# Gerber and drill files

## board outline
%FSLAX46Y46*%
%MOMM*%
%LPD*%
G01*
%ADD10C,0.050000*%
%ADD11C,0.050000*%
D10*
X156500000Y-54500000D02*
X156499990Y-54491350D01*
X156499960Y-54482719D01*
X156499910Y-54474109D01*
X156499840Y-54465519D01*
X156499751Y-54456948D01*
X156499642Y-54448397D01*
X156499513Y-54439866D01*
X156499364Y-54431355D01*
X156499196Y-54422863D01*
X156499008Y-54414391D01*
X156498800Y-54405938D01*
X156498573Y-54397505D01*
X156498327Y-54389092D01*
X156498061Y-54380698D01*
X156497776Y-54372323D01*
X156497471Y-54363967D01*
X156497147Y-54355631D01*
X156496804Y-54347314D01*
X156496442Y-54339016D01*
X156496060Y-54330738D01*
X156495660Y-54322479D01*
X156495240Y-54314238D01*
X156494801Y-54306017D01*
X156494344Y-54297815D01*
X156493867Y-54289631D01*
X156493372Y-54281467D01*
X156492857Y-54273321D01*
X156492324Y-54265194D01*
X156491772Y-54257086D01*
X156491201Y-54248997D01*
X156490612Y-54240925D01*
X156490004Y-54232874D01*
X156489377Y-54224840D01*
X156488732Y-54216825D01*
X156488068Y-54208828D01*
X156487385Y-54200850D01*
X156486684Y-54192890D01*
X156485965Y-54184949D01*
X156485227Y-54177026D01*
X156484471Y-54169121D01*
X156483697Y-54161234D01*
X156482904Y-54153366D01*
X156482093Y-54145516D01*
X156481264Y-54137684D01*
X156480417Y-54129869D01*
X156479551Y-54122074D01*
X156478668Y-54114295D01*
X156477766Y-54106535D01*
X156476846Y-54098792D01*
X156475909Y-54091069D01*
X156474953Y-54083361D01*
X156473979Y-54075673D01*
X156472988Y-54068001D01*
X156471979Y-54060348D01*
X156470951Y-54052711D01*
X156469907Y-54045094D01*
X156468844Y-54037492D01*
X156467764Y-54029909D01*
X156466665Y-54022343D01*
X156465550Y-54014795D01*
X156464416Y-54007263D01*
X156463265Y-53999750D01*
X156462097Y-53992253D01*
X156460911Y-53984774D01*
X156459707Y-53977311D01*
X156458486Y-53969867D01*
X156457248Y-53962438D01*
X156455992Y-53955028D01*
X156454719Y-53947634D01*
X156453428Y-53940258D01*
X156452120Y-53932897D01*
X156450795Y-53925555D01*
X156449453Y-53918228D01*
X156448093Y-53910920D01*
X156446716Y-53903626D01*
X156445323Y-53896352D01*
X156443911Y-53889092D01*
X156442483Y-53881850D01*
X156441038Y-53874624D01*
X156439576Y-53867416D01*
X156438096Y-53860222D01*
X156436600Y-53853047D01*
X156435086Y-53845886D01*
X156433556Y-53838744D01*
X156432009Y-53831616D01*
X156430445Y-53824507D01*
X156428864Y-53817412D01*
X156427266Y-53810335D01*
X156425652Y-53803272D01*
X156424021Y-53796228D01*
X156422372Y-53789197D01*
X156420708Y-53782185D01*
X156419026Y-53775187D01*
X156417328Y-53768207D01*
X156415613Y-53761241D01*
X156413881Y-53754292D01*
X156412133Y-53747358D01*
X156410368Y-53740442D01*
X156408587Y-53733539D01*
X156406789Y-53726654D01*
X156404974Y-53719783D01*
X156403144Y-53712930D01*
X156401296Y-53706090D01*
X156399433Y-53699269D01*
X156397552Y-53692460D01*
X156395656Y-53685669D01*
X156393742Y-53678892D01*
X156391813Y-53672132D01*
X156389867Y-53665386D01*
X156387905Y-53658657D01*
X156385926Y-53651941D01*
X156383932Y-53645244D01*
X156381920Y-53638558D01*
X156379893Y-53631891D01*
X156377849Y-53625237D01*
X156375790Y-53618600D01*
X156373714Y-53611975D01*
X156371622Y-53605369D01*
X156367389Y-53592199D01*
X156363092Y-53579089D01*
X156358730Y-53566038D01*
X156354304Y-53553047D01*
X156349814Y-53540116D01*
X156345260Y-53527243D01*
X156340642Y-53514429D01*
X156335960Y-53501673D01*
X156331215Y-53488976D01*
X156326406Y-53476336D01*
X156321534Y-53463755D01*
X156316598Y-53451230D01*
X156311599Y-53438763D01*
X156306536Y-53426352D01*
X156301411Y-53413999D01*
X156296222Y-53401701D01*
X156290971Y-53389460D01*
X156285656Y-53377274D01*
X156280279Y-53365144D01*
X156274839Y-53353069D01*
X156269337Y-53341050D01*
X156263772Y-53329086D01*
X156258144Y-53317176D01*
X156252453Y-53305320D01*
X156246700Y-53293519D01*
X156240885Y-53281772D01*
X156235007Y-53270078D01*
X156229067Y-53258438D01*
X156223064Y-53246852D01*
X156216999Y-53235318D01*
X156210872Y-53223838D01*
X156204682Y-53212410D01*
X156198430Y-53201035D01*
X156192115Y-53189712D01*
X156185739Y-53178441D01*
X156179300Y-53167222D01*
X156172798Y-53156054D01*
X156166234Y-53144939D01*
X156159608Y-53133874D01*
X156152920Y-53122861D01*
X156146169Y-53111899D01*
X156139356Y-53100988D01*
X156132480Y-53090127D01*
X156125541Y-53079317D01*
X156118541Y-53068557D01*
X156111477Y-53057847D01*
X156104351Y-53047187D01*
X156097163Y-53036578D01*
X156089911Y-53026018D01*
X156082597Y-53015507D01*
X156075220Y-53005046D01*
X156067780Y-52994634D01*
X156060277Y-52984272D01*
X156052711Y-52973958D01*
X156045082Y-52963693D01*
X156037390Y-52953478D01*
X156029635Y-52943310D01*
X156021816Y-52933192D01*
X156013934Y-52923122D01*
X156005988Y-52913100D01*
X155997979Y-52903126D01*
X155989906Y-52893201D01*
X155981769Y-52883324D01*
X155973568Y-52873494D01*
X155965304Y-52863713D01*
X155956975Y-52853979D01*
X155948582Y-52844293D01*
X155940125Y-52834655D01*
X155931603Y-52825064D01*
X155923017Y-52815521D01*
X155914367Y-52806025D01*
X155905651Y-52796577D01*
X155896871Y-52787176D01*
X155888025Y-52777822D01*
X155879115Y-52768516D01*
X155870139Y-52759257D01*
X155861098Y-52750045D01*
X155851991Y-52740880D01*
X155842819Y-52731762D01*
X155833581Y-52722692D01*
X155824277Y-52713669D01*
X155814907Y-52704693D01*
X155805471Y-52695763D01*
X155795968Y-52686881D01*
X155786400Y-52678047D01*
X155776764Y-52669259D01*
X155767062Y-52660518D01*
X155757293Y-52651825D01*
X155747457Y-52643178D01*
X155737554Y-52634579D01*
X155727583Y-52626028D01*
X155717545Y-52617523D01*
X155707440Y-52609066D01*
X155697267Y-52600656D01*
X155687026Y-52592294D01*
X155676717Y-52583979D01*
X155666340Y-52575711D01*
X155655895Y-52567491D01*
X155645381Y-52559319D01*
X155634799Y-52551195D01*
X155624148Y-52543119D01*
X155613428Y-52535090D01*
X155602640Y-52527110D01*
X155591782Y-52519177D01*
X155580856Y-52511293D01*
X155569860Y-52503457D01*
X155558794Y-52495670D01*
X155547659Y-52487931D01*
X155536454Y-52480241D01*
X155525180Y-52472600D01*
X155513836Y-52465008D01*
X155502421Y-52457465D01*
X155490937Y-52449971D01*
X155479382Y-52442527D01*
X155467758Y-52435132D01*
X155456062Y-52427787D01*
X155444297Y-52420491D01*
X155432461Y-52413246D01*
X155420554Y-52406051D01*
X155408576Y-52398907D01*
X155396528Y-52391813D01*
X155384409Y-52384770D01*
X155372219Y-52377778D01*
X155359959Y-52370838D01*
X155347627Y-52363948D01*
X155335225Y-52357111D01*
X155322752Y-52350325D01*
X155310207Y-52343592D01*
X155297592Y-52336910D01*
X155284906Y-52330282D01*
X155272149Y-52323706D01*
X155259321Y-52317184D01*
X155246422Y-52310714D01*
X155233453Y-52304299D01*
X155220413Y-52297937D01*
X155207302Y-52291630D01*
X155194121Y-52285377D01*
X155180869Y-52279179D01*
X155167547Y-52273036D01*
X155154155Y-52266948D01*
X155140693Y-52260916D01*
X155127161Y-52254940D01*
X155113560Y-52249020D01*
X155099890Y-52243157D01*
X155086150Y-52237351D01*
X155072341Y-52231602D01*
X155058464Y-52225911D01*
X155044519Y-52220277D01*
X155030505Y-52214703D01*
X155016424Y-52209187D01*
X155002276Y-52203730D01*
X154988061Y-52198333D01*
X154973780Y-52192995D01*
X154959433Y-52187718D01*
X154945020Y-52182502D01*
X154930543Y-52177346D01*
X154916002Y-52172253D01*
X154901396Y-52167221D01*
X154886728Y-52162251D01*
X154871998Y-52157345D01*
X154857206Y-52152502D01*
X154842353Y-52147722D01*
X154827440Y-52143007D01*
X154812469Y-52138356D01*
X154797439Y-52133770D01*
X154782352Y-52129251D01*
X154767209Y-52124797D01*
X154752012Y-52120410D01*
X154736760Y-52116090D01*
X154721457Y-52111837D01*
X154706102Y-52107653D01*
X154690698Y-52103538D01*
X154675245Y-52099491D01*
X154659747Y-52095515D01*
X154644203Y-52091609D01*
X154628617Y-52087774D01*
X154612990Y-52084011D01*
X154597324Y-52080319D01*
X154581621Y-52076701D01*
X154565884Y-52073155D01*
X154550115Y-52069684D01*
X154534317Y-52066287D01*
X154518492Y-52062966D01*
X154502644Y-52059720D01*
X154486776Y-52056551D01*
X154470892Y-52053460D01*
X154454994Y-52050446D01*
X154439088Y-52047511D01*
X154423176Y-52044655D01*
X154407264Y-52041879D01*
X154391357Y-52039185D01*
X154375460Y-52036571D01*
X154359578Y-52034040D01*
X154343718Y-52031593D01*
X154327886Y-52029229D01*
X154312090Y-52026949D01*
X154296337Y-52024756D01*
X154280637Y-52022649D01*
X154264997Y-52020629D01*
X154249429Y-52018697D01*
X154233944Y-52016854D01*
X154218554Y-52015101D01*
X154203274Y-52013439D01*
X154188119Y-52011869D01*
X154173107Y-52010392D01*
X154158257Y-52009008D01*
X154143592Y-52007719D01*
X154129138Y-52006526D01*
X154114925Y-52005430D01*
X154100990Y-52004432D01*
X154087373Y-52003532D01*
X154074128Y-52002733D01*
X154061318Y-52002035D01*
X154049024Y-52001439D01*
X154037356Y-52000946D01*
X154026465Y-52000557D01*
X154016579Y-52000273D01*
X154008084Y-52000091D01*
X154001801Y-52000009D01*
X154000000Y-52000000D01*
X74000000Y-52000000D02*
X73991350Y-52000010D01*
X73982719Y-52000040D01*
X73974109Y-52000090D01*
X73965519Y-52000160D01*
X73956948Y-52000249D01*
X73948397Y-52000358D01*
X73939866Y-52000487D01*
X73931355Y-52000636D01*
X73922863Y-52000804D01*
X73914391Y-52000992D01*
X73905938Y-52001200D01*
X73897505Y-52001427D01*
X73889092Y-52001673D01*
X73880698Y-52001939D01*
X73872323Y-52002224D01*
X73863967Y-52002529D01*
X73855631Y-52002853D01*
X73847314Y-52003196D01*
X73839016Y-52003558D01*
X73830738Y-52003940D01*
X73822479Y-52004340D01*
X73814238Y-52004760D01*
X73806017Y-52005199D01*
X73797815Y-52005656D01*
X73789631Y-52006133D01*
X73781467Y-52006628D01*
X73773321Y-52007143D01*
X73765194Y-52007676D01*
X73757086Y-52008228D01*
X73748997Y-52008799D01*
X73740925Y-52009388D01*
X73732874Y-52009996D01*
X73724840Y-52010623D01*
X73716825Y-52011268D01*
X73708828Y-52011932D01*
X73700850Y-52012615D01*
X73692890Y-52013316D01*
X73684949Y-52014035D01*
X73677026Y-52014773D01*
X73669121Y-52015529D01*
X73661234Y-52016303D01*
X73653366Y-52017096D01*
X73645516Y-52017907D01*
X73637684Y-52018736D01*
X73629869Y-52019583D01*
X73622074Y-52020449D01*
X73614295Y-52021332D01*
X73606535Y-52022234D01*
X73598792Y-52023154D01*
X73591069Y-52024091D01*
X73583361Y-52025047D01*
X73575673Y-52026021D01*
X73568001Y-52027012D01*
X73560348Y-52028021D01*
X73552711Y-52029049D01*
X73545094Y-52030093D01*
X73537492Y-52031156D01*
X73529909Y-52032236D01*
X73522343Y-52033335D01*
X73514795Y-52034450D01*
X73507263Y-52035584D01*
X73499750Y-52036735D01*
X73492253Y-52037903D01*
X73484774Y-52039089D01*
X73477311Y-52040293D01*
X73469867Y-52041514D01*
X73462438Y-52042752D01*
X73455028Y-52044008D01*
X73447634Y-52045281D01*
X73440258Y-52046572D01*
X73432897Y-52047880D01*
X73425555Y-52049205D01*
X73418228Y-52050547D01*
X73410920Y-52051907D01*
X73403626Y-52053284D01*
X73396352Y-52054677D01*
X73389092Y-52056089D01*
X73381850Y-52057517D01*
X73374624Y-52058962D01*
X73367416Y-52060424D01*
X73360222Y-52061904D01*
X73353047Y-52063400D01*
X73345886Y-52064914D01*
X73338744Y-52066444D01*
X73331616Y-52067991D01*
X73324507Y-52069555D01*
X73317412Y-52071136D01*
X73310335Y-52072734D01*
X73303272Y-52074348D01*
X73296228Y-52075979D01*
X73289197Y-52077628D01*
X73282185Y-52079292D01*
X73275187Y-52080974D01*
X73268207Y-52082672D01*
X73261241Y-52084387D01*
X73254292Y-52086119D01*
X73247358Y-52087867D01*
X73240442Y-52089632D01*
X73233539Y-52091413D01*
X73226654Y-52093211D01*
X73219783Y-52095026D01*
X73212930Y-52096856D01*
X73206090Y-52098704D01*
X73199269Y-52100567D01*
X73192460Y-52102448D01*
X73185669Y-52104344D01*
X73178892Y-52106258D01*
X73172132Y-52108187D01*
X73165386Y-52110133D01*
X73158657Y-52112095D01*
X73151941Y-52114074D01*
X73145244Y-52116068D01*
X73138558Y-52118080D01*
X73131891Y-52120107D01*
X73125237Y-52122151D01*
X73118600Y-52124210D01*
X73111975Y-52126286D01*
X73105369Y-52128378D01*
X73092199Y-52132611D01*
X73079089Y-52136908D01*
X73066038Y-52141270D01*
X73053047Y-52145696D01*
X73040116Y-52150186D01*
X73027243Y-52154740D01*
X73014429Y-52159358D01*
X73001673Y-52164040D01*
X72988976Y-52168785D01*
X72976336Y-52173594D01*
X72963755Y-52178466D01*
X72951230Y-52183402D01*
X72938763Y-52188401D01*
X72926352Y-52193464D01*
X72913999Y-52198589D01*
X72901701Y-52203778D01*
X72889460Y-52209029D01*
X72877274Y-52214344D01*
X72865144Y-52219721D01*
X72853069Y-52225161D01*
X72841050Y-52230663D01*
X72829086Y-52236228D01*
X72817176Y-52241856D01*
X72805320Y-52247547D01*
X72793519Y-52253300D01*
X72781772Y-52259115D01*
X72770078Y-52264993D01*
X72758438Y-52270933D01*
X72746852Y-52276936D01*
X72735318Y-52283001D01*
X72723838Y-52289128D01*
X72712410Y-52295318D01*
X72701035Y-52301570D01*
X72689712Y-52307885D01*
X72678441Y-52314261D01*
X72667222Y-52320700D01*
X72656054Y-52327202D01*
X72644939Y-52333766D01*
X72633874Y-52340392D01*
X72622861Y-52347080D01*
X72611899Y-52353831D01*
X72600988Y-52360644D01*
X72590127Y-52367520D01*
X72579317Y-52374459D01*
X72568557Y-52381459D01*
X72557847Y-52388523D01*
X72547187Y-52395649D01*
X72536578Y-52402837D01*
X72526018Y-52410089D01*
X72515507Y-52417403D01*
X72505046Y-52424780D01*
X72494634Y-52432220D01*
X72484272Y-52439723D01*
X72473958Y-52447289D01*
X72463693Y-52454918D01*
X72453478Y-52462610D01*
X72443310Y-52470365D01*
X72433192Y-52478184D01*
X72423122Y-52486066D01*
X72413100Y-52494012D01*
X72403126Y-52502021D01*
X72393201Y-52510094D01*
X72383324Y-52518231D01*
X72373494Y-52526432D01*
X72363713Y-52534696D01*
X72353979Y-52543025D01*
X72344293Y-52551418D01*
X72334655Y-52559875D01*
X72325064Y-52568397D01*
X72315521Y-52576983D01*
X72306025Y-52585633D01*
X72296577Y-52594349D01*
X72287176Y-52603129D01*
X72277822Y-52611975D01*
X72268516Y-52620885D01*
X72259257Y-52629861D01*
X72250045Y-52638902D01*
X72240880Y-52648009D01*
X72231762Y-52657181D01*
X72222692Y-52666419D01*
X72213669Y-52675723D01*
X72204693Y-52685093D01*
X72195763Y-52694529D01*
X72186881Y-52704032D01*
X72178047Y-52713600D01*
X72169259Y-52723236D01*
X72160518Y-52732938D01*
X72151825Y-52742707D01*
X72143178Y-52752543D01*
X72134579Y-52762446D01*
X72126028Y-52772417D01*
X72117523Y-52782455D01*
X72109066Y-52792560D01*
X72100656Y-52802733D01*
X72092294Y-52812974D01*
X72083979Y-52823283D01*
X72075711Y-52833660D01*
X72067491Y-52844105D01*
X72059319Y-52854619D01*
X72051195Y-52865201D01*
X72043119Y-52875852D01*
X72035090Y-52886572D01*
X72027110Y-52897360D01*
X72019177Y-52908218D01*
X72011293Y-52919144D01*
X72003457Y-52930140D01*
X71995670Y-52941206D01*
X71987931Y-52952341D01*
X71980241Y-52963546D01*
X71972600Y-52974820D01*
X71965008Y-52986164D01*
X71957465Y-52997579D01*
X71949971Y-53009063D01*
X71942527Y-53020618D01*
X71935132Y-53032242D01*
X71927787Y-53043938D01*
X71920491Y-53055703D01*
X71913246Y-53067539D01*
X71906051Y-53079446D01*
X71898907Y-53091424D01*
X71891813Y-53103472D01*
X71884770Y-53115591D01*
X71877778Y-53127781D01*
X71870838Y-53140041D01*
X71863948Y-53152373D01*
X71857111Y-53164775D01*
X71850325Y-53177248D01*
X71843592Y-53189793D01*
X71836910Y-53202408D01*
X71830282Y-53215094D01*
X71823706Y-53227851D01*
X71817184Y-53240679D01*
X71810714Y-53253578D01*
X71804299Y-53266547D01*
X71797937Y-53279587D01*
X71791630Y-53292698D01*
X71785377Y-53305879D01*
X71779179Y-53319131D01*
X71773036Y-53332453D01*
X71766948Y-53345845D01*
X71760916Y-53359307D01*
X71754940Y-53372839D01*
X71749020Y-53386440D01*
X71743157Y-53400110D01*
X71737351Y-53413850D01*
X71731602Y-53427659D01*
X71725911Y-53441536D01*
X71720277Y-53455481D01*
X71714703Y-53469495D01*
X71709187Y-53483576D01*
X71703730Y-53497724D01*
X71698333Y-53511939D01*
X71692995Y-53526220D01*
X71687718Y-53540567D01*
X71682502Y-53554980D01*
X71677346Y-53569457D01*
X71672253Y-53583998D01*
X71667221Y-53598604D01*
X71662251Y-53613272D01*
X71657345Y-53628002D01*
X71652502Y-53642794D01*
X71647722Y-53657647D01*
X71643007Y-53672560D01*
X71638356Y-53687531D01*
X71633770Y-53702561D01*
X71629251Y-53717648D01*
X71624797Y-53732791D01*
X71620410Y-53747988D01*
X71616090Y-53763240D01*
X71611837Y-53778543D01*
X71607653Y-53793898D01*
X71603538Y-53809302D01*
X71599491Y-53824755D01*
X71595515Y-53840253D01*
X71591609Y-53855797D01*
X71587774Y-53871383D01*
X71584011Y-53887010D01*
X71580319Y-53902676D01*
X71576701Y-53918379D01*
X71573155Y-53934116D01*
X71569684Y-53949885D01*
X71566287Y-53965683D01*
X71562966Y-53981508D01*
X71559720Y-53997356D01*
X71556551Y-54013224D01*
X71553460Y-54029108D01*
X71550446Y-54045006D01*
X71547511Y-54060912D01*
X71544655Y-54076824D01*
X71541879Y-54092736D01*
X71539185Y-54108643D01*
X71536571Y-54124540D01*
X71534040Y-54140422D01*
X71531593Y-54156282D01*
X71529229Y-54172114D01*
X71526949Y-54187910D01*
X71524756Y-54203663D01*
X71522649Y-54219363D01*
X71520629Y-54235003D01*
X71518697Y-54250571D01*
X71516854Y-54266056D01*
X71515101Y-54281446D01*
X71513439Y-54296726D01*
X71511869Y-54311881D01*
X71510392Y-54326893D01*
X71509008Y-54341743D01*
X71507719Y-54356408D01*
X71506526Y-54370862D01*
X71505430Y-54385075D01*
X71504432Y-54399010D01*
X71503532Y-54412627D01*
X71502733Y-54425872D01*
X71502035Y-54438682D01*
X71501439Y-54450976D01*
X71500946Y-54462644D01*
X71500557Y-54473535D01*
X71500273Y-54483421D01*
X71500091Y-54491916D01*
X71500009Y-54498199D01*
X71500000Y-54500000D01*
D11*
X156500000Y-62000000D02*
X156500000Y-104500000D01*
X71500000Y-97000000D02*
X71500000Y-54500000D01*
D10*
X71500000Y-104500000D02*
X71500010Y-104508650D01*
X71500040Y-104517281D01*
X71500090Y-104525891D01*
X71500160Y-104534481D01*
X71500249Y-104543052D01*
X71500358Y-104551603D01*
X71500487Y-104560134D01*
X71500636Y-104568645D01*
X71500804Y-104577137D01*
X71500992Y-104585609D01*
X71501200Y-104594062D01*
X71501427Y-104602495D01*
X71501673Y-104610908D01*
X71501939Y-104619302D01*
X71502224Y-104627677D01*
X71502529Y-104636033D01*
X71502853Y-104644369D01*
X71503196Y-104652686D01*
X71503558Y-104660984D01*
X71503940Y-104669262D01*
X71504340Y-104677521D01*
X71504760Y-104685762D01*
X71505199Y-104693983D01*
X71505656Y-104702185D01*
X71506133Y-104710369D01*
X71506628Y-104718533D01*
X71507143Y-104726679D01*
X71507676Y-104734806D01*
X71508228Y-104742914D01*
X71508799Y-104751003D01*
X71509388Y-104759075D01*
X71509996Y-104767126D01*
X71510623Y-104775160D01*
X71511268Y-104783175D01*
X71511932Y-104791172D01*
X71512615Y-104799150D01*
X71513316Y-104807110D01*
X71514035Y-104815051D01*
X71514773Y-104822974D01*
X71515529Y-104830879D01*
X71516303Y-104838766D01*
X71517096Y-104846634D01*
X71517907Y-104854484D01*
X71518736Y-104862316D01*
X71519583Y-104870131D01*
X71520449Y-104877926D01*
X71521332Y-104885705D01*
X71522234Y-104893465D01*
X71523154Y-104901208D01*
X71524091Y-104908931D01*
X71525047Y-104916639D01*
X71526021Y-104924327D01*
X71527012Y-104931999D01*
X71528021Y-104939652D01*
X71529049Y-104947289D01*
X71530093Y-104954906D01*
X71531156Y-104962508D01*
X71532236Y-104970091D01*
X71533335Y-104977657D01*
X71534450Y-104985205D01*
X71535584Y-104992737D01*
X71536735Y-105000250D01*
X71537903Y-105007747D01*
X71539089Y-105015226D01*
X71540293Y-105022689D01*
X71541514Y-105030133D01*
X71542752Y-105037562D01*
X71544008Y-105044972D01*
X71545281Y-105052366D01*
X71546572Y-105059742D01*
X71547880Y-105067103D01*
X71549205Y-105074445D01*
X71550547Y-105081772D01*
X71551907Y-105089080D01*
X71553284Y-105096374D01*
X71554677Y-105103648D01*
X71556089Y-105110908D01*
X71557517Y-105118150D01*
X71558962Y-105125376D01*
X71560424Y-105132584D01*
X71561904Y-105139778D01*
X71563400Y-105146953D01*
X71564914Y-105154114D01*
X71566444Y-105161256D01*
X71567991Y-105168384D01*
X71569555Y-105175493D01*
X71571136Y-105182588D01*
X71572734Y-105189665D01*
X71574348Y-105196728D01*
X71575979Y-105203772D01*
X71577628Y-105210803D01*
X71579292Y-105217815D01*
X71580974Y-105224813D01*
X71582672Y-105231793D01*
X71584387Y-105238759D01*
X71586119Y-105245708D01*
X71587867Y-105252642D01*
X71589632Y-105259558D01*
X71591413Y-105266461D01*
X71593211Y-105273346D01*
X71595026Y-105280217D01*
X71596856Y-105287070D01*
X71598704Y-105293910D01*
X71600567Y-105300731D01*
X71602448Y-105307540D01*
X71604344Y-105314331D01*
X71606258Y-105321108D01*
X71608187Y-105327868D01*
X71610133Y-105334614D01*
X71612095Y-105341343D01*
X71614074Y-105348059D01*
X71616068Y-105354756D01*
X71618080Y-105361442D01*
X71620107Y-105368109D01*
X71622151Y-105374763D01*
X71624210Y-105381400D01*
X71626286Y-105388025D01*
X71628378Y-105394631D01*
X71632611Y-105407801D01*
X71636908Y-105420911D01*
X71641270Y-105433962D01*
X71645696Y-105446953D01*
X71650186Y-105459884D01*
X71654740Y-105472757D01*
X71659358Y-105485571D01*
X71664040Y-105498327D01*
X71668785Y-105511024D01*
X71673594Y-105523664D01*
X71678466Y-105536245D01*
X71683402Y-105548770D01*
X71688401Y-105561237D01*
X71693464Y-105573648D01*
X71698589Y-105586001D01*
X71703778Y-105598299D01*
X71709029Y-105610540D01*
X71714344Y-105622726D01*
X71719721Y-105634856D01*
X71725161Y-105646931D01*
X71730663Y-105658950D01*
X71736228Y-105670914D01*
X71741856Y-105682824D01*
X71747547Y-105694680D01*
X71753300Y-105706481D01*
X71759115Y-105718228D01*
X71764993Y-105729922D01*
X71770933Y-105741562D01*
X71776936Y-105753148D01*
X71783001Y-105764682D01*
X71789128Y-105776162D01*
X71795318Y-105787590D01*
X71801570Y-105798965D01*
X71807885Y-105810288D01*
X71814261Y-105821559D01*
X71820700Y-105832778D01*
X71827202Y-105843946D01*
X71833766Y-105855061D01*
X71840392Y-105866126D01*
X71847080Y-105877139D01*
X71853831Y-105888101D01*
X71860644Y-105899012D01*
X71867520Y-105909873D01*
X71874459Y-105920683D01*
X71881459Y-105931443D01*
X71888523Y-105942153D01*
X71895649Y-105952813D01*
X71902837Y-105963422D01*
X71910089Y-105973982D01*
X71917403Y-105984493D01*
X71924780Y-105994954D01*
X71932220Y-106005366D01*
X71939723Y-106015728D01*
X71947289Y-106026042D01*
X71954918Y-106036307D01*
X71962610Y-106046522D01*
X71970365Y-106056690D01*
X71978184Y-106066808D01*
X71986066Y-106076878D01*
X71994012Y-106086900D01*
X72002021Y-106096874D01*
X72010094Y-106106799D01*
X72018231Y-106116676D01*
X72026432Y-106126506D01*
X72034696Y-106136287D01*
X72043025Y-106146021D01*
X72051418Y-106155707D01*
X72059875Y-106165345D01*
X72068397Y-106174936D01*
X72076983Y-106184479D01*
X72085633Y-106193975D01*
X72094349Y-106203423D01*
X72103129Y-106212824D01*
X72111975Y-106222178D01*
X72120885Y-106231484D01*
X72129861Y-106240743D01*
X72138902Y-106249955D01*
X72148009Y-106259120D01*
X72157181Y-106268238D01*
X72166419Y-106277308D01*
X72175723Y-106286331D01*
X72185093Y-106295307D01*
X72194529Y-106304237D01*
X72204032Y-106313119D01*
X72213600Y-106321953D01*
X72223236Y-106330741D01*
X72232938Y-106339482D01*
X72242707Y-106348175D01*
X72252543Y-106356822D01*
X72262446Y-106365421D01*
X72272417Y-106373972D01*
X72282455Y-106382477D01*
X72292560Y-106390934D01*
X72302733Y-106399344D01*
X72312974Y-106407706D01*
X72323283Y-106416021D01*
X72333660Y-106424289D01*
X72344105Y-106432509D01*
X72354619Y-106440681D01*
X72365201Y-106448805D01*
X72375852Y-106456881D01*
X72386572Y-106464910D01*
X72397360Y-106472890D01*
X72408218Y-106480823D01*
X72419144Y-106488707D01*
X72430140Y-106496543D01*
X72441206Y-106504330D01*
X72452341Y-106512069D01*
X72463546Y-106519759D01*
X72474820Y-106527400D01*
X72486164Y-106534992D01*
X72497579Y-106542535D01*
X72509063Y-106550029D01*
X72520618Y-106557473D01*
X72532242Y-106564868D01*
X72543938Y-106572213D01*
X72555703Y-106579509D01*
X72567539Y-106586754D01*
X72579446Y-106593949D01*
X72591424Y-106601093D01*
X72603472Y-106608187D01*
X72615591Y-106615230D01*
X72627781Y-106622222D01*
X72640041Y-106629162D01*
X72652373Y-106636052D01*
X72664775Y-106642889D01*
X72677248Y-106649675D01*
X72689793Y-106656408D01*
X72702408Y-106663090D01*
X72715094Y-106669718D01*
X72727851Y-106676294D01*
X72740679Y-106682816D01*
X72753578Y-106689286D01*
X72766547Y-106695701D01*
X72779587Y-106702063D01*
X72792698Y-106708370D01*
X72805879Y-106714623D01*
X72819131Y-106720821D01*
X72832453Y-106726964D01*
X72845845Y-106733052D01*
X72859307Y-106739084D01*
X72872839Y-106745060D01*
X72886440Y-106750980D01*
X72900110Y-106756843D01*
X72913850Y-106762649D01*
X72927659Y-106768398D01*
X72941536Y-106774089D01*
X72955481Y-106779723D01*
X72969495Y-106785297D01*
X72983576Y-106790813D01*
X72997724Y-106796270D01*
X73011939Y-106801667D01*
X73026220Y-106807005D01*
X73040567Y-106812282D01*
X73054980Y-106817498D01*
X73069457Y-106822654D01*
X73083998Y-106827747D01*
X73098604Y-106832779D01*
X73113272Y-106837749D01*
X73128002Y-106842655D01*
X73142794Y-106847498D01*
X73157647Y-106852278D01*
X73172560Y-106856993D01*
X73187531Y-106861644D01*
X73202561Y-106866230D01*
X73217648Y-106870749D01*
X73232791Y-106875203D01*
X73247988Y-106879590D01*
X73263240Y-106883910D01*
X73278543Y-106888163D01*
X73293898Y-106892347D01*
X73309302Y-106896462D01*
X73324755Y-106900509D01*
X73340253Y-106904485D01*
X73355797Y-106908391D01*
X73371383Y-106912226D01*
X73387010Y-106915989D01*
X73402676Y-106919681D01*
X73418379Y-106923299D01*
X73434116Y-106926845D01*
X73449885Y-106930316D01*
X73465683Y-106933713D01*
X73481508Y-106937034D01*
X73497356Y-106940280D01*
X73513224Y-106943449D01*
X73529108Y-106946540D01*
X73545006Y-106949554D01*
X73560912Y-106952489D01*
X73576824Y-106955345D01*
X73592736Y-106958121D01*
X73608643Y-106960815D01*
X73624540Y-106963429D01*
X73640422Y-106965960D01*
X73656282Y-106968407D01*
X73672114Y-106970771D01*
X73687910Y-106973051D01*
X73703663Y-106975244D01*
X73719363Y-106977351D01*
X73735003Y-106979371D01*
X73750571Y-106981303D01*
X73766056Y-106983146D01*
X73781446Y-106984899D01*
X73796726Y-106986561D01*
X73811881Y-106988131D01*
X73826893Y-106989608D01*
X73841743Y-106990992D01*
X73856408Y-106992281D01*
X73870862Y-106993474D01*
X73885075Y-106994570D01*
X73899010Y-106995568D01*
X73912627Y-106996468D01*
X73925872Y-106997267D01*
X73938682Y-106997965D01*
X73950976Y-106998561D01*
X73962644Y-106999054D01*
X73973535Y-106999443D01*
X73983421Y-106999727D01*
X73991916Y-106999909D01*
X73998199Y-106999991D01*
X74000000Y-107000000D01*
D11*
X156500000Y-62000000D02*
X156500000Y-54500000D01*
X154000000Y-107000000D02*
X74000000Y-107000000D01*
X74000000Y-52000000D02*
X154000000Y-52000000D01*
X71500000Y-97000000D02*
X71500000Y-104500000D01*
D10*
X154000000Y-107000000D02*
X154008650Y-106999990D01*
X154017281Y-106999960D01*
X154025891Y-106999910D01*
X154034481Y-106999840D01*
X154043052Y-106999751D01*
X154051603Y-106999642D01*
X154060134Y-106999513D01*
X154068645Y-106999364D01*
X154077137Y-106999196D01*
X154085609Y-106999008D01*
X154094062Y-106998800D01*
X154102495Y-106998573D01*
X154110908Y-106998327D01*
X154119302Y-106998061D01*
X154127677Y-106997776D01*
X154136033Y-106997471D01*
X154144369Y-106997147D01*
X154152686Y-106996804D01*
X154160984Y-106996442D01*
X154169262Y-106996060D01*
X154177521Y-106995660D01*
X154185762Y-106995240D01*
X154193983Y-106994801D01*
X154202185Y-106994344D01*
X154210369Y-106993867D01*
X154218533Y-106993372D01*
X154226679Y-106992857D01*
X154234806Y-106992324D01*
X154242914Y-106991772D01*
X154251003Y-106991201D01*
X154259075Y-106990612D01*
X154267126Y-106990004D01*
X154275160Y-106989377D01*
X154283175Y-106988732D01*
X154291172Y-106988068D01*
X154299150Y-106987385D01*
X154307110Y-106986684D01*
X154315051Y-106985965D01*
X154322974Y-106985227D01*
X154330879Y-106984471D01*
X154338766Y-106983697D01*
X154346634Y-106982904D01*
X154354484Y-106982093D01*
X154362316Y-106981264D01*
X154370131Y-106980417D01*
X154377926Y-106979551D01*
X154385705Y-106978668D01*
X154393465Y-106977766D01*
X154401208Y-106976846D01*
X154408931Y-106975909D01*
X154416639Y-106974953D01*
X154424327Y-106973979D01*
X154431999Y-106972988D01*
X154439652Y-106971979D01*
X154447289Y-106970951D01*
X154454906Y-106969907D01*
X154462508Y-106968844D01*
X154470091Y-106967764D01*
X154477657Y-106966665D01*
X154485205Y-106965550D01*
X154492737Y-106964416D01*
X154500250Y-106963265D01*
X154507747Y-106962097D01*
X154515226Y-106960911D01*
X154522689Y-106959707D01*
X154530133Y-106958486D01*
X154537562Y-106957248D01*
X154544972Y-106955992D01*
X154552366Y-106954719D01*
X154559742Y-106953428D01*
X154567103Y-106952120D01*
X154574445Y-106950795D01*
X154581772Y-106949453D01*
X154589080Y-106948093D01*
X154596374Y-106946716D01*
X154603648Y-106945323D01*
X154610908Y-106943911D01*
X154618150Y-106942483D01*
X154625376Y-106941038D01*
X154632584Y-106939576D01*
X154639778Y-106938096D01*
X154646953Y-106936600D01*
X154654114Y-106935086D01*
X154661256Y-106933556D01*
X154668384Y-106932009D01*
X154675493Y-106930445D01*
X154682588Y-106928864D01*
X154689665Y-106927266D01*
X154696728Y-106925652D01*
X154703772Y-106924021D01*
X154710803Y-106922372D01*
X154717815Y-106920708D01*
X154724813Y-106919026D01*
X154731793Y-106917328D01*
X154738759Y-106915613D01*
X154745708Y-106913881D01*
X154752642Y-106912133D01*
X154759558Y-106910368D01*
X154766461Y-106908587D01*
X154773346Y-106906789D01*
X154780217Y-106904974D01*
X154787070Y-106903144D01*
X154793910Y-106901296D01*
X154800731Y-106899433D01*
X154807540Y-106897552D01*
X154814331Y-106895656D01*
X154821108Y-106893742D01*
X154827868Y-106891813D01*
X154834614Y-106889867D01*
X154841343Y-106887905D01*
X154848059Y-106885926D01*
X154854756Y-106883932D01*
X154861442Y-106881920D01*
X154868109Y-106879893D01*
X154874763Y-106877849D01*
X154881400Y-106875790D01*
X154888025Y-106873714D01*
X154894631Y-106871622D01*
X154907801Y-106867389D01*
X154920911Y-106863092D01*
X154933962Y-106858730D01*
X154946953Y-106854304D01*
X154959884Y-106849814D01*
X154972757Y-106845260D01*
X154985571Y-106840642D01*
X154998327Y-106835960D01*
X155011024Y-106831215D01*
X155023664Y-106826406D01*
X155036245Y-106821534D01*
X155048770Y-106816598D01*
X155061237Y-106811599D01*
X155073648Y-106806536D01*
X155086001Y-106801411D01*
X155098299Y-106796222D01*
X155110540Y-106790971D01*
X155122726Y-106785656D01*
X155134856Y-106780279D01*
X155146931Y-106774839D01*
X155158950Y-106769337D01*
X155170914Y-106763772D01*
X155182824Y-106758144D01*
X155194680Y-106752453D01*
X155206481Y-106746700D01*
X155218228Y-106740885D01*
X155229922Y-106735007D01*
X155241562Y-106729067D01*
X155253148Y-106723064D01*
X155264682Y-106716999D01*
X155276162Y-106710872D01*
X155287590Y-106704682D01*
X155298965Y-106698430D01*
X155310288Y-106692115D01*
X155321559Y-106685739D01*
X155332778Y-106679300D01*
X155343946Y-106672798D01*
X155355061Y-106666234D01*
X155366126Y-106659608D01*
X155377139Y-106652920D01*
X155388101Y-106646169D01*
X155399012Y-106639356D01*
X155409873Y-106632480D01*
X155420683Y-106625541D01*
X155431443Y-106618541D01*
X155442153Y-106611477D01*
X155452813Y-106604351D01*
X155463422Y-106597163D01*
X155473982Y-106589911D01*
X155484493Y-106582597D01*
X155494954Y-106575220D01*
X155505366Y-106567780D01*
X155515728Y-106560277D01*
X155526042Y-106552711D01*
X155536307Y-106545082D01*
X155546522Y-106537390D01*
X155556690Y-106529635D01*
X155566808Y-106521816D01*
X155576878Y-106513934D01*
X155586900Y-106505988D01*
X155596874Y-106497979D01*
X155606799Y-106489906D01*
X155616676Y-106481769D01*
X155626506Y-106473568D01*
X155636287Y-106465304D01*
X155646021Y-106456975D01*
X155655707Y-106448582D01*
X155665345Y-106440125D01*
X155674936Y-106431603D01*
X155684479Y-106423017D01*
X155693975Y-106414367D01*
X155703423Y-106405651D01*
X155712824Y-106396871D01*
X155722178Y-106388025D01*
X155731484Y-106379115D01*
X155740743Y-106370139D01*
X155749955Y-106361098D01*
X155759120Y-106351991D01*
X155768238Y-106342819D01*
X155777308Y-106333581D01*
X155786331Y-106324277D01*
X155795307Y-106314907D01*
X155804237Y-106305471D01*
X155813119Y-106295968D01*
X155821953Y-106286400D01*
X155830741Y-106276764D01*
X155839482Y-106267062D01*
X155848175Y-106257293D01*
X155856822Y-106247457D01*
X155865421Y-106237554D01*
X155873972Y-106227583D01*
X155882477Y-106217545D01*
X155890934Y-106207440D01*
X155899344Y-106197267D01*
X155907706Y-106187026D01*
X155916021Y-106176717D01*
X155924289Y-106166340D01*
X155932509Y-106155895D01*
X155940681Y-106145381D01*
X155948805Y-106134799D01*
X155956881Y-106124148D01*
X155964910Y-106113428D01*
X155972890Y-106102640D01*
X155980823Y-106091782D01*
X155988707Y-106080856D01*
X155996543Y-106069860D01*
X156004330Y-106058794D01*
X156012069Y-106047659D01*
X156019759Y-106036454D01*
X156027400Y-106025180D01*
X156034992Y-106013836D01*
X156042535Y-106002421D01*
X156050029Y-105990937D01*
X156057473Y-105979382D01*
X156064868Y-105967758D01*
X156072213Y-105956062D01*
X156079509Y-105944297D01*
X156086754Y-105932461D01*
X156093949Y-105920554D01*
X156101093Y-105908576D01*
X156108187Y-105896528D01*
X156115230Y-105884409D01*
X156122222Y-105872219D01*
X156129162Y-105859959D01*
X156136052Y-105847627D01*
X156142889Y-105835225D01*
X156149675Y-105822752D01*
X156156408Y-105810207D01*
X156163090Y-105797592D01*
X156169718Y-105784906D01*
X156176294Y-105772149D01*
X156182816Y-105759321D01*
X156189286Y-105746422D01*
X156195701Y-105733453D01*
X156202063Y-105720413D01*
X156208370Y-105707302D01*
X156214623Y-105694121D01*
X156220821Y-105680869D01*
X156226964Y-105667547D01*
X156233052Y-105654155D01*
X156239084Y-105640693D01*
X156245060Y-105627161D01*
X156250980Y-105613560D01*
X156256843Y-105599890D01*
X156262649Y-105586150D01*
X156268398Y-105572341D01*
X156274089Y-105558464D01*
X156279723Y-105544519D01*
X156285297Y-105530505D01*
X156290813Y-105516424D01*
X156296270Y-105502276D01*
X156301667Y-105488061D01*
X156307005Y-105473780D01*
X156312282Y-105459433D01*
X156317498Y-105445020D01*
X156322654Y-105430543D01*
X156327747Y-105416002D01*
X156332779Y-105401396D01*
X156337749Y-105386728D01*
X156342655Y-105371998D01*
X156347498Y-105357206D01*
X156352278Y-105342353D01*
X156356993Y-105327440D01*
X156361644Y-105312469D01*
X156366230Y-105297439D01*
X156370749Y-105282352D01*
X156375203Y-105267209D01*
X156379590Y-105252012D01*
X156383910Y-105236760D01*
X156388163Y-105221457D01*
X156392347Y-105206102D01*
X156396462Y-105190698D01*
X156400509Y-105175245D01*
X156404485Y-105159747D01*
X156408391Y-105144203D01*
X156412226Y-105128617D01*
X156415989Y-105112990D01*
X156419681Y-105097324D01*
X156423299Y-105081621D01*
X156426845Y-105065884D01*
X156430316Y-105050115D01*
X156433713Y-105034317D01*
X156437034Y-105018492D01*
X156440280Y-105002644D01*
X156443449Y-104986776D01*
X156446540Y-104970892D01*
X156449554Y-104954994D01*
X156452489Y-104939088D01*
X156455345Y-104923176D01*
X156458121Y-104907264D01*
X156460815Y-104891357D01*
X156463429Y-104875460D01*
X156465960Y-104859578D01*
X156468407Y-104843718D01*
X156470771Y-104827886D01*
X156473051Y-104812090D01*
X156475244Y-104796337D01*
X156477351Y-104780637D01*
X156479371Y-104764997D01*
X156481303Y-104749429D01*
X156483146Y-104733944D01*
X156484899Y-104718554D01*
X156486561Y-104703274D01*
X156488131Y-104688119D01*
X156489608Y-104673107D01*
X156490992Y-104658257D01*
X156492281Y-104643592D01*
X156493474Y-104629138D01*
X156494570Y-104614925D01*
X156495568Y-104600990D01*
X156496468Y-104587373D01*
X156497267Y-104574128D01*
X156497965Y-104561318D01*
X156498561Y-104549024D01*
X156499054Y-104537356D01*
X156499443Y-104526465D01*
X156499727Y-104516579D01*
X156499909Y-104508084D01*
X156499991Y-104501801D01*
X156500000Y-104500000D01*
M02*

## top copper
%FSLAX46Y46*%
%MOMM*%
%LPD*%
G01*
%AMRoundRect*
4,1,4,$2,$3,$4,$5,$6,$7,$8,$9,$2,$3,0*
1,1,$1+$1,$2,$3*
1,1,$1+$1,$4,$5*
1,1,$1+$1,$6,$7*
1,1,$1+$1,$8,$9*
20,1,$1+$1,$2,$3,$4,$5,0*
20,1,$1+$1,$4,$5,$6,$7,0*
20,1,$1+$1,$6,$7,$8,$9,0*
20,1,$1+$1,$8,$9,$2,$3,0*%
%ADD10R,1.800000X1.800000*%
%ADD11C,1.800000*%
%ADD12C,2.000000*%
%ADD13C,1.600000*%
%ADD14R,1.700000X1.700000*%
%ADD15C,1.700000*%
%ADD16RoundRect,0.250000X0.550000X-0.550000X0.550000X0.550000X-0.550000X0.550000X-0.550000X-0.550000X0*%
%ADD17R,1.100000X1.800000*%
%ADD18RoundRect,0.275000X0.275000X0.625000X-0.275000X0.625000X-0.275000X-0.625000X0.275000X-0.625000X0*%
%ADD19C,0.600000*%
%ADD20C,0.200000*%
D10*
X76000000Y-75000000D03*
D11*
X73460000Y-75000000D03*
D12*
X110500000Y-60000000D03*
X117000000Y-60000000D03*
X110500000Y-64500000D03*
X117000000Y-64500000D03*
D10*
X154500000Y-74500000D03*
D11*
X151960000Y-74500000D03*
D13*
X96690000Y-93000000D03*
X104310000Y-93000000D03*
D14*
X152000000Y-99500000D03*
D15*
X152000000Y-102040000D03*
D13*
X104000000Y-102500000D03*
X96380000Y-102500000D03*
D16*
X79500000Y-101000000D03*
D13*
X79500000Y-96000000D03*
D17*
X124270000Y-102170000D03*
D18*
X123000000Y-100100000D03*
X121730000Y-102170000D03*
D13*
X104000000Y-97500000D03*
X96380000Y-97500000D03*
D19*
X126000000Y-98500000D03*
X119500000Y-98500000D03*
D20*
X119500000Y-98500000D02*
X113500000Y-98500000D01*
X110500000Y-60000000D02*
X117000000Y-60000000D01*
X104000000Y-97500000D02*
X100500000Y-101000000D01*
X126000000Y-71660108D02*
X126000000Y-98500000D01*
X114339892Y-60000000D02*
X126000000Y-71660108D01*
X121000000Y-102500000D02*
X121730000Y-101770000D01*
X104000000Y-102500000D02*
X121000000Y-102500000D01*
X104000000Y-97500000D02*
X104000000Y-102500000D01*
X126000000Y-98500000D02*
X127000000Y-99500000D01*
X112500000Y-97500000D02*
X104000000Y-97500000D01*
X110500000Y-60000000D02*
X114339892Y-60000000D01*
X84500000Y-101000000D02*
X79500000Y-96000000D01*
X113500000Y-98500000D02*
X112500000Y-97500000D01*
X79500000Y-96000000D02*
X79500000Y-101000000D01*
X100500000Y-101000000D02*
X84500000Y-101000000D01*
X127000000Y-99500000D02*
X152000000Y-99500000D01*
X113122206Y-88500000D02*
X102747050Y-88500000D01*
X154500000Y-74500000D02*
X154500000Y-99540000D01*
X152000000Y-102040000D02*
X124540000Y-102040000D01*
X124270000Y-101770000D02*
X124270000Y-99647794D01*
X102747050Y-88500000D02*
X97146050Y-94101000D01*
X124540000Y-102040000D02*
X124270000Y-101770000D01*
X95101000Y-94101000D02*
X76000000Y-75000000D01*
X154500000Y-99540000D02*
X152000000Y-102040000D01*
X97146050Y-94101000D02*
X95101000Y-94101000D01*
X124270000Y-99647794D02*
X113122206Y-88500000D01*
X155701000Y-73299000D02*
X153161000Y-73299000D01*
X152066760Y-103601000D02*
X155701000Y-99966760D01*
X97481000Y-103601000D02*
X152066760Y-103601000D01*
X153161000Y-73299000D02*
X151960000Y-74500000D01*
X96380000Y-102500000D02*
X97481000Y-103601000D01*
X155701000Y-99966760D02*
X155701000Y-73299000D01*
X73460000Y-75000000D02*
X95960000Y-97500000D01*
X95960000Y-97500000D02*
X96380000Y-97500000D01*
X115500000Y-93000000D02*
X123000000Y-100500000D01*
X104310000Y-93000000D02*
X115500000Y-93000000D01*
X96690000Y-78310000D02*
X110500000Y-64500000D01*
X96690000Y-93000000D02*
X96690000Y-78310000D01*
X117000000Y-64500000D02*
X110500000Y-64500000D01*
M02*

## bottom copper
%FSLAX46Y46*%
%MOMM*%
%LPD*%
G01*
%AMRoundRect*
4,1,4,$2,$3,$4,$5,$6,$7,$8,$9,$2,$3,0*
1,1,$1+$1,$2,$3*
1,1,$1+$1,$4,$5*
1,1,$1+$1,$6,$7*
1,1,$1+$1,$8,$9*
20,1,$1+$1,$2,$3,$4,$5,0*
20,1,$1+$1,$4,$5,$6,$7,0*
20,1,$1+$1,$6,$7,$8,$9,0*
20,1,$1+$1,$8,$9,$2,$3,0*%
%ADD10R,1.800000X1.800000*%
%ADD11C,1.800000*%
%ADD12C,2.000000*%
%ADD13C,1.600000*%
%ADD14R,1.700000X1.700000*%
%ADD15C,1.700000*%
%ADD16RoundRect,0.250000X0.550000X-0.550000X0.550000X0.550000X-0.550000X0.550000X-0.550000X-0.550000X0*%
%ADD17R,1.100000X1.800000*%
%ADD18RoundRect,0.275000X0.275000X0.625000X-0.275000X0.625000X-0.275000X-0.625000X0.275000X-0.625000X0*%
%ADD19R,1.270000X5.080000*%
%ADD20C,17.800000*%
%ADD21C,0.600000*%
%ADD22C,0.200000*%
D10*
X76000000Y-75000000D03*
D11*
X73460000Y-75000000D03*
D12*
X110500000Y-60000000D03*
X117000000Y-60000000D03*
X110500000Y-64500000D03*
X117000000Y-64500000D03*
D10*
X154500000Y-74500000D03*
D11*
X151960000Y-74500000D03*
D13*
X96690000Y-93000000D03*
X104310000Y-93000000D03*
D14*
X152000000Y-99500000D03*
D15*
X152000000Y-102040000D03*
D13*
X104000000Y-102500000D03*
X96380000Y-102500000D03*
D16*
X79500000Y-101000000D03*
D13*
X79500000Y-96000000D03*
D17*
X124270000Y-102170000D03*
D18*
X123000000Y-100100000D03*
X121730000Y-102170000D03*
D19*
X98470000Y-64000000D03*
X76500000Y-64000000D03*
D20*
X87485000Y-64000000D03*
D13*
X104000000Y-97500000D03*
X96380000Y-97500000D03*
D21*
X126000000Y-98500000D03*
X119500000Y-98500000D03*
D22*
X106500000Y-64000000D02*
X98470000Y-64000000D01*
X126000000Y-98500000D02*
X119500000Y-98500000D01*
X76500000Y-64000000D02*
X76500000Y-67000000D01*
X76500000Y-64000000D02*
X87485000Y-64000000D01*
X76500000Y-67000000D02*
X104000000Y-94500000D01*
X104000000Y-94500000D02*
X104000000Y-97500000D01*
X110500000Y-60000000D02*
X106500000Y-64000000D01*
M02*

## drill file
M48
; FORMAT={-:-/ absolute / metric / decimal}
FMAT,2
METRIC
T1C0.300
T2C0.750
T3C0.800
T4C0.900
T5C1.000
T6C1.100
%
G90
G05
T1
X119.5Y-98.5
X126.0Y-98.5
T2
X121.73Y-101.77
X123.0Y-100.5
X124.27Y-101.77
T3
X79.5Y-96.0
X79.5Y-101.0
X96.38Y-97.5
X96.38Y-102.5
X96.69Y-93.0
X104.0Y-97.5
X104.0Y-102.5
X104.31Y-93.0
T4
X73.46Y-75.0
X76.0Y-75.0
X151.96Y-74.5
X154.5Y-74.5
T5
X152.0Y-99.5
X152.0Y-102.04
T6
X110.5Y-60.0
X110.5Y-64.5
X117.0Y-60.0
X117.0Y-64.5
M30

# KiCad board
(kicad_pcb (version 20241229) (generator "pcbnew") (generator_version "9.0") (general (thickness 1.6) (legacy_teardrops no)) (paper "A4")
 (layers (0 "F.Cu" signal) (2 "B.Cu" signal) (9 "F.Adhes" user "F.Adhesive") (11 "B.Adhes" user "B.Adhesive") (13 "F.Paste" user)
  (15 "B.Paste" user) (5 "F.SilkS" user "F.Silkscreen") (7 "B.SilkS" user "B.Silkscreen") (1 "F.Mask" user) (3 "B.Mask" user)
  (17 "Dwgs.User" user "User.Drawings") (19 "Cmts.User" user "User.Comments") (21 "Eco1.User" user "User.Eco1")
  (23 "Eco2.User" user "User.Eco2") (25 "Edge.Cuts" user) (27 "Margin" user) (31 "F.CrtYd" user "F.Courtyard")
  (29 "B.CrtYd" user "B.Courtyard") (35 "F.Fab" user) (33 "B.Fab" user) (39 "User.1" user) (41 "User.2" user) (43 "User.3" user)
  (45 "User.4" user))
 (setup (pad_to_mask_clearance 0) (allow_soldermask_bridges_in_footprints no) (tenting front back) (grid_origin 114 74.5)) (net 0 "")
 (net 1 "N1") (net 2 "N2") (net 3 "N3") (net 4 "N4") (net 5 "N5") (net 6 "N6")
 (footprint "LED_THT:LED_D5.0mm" (layer "F.Cu") (at 76 75 180)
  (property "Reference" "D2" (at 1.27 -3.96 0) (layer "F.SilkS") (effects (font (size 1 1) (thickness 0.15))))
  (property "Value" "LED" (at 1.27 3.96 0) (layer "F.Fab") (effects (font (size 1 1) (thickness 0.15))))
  (pad "1" thru_hole rect (at 0 0 180) (size 1.8 1.8) (drill 0.9) (layers "*.Cu" "*.Mask") (remove_unused_layers no) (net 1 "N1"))
  (pad "2" thru_hole circle (at 2.54 0 180) (size 1.8 1.8) (drill 0.9) (layers "*.Cu" "*.Mask") (remove_unused_layers no) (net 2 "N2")))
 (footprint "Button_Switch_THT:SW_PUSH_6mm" (layer "F.Cu") (at 110.5 60)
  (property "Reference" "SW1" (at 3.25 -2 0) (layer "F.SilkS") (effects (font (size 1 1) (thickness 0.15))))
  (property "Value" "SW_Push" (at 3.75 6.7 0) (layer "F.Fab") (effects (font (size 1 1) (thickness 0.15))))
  (pad "1" thru_hole circle (at 0 0 90) (size 2 2) (drill 1.1) (layers "*.Cu" "*.Mask") (remove_unused_layers no) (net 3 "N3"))
  (pad "1" thru_hole circle (at 6.5 0 90) (size 2 2) (drill 1.1) (layers "*.Cu" "*.Mask") (remove_unused_layers no) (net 3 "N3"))
  (pad "2" thru_hole circle (at 0 4.5 90) (size 2 2) (drill 1.1) (layers "*.Cu" "*.Mask") (remove_unused_layers no) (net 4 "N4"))
  (pad "2" thru_hole circle (at 6.5 4.5 90) (size 2 2) (drill 1.1) (layers "*.Cu" "*.Mask") (remove_unused_layers no) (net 4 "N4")))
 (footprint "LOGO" (layer "F.Cu") (at 139 88.5)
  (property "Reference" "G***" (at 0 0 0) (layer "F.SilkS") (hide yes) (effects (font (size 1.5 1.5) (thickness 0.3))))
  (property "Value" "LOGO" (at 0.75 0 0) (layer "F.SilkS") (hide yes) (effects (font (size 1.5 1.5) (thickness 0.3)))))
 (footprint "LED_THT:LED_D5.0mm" (layer "F.Cu") (at 154.5 74.5 180)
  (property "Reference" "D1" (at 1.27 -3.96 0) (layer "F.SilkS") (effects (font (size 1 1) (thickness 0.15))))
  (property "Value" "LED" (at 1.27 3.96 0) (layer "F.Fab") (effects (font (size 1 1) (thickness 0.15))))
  (pad "1" thru_hole rect (at 0 0 180) (size 1.8 1.8) (drill 0.9) (layers "*.Cu" "*.Mask") (remove_unused_layers no) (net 1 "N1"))
  (pad "2" thru_hole circle (at 2.54 0 180) (size 1.8 1.8) (drill 0.9) (layers "*.Cu" "*.Mask") (remove_unused_layers no) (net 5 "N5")))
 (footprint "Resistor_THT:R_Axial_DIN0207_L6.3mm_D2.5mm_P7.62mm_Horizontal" (layer "B.Cu") (at 96.69 93)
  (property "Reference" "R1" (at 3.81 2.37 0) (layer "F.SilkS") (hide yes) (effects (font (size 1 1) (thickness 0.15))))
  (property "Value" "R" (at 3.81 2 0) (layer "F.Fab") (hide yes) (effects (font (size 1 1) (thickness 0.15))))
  (pad "1" thru_hole circle (at 0 0) (size 1.6 1.6) (drill 0.8) (layers "*.Cu" "*.Mask") (remove_unused_layers no) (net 4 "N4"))
  (pad "2" thru_hole circle (at 7.62 0) (size 1.6 1.6) (drill 0.8) (layers "*.Cu" "*.Mask") (remove_unused_layers no) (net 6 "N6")))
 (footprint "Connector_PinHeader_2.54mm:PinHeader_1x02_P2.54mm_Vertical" (layer "B.Cu") (at 152 99.5 180)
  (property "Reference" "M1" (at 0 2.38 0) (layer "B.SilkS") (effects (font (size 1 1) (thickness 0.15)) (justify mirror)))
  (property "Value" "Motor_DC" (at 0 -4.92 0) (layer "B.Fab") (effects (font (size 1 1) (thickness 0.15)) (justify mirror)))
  (pad "1" thru_hole rect (at 0 0 180) (size 1.7 1.7) (drill 1) (layers "*.Cu" "*.Mask") (remove_unused_layers no) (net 3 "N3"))
  (pad "2" thru_hole circle (at 0 -2.54 180) (size 1.7 1.7) (drill 1) (layers "*.Cu" "*.Mask") (remove_unused_layers no) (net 1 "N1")))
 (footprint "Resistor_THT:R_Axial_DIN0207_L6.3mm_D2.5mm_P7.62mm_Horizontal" (layer "B.Cu") (at 104 102.5 180)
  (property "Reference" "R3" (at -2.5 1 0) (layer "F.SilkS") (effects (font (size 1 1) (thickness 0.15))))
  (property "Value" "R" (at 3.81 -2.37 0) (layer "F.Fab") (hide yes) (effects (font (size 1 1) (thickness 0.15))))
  (pad "1" thru_hole circle (at 0 0 180) (size 1.6 1.6) (drill 0.8) (layers "*.Cu" "*.Mask") (remove_unused_layers no) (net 3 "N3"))
  (pad "2" thru_hole circle (at 7.62 0 180) (size 1.6 1.6) (drill 0.8) (layers "*.Cu" "*.Mask") (remove_unused_layers no) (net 5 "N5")))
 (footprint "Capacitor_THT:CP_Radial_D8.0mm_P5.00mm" (layer "B.Cu") (at 79.5 101 90)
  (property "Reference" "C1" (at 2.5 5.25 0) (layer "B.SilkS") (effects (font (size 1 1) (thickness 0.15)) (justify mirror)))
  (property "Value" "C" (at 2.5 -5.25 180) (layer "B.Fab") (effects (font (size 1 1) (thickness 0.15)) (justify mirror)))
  (pad "1" thru_hole roundrect (at 0 0 90) (size 1.6 1.6) (drill 0.8) (layers "*.Cu" "*.Mask") (remove_unused_layers no)
   (roundrect_rratio 0.15625) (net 3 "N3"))
  (pad "2" thru_hole circle (at 5 0 90) (size 1.6 1.6) (drill 0.8) (layers "*.Cu" "*.Mask") (remove_unused_layers no) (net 3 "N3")))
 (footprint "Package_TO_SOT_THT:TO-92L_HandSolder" (layer "B.Cu") (at 124.27 101.77 180)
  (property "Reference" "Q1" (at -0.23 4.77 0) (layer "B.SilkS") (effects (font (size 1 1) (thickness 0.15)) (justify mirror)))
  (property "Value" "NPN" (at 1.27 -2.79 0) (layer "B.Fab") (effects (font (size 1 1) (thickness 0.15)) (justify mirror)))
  (pad "1" thru_hole rect (at 0 0 180) (size 1.1 1.8) (drill 0.75 (offset 0 -0.4)) (layers "*.Cu" "*.Mask") (remove_unused_layers no)
   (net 1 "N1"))
  (pad "2" thru_hole roundrect (at 1.27 1.27 180) (size 1.1 1.8) (drill 0.75 (offset 0 0.4)) (layers "*.Cu" "*.Mask")
   (remove_unused_layers no) (roundrect_rratio 0.25) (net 6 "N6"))
  (pad "3" thru_hole roundrect (at 2.54 0 180) (size 1.1 1.8) (drill 0.75 (offset 0 -0.4)) (layers "*.Cu" "*.Mask")
   (remove_unused_layers no) (roundrect_rratio 0.25) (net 3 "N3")))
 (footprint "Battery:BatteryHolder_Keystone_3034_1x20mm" (layer "B.Cu") (at 87.485 64 180)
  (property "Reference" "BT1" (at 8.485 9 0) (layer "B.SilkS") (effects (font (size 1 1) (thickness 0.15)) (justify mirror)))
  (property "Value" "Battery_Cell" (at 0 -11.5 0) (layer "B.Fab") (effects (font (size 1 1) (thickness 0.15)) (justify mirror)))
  (pad "1" smd rect (at -10.985 0 180) (size 1.27 5.08) (layers "B.Cu" "B.Mask" "B.Paste") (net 3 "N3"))
  (pad "1" smd rect (at 10.985 0 180) (size 1.27 5.08) (layers "B.Cu" "B.Mask" "B.Paste") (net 3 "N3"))
  (pad "2" smd circle (at 0 0 180) (size 17.8 17.8) (layers "B.Cu" "B.Mask") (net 3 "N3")))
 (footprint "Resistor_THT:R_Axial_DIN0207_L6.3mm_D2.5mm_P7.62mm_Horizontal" (layer "B.Cu") (at 104 97.5 180)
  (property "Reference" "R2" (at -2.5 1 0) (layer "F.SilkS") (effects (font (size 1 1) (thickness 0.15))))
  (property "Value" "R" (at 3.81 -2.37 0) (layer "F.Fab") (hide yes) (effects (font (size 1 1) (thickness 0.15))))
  (pad "1" thru_hole circle (at 0 0 180) (size 1.6 1.6) (drill 0.8) (layers "*.Cu" "*.Mask") (remove_unused_layers no) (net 3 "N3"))
  (pad "2" thru_hole circle (at 7.62 0 180) (size 1.6 1.6) (drill 0.8) (layers "*.Cu" "*.Mask") (remove_unused_layers no) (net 2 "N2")))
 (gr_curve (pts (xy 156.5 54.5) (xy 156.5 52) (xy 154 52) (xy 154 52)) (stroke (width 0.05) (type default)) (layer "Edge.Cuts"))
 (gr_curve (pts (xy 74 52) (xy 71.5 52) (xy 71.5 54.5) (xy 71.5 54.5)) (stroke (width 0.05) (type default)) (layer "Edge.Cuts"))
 (gr_line (start 156.5 62) (end 156.5 104.5) (stroke (width 0.05) (type default)) (layer "Edge.Cuts"))
 (gr_line (start 71.5 97) (end 71.5 54.5) (stroke (width 0.05) (type default)) (layer "Edge.Cuts"))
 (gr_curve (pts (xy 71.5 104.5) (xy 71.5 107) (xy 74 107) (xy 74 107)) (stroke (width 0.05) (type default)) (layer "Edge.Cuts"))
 (gr_line (start 156.5 62) (end 156.5 54.5) (stroke (width 0.05) (type default)) (layer "Edge.Cuts"))
 (gr_line (start 154 107) (end 74 107) (stroke (width 0.05) (type default)) (layer "Edge.Cuts"))
 (gr_line (start 74 52) (end 154 52) (stroke (width 0.05) (type default)) (layer "Edge.Cuts"))
 (gr_line (start 71.5 97) (end 71.5 104.5) (stroke (width 0.05) (type default)) (layer "Edge.Cuts"))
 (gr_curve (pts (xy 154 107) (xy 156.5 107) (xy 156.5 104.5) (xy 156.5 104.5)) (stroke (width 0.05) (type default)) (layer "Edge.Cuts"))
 (segment (start 119.5 98.5) (end 113.5 98.5) (width 0.2) (layer "F.Cu") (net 3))
 (segment (start 110.5 60) (end 117 60) (width 0.2) (layer "F.Cu") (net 3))
 (segment (start 104 97.5) (end 100.5 101) (width 0.2) (layer "F.Cu") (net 3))
 (segment (start 126 71.660108) (end 126 98.5) (width 0.2) (layer "F.Cu") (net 3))
 (segment (start 114.339892 60) (end 126 71.660108) (width 0.2) (layer "F.Cu") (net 3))
 (segment (start 121 102.5) (end 121.73 101.77) (width 0.2) (layer "F.Cu") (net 3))
 (segment (start 104 102.5) (end 121 102.5) (width 0.2) (layer "F.Cu") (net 3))
 (segment (start 104 97.5) (end 104 102.5) (width 0.2) (layer "F.Cu") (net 3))
 (segment (start 126 98.5) (end 127 99.5) (width 0.2) (layer "F.Cu") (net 3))
 (segment (start 112.5 97.5) (end 104 97.5) (width 0.2) (layer "F.Cu") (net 3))
 (segment (start 110.5 60) (end 114.339892 60) (width 0.2) (layer "F.Cu") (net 3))
 (segment (start 84.5 101) (end 79.5 96) (width 0.2) (layer "F.Cu") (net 3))
 (segment (start 113.5 98.5) (end 112.5 97.5) (width 0.2) (layer "F.Cu") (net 3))
 (segment (start 79.5 96) (end 79.5 101) (width 0.2) (layer "F.Cu") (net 3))
 (segment (start 100.5 101) (end 84.5 101) (width 0.2) (layer "F.Cu") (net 3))
 (segment (start 127 99.5) (end 152 99.5) (width 0.2) (layer "F.Cu") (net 3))
 (via (at 126 98.5) (size 0.6) (drill 0.3) (layers "F.Cu" "B.Cu") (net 3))
 (via (at 119.5 98.5) (size 0.6) (drill 0.3) (layers "F.Cu" "B.Cu") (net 3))
 (segment (start 106.5 64) (end 98.47 64) (width 0.2) (layer "B.Cu") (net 3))
 (segment (start 126 98.5) (end 119.5 98.5) (width 0.2) (layer "B.Cu") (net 3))
 (segment (start 76.5 64) (end 76.5 67) (width 0.2) (layer "B.Cu") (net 3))
 (segment (start 76.5 64) (end 87.485 64) (width 0.2) (layer "B.Cu") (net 3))
 (segment (start 76.5 67) (end 104 94.5) (width 0.2) (layer "B.Cu") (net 3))
 (segment (start 104 94.5) (end 104 97.5) (width 0.2) (layer "B.Cu") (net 3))
 (segment (start 110.5 60) (end 106.5 64) (width 0.2) (layer "B.Cu") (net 3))
 (segment (start 113.122206 88.5) (end 102.74705 88.5) (width 0.2) (layer "F.Cu") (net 1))
 (segment (start 154.5 74.5) (end 154.5 99.54) (width 0.2) (layer "F.Cu") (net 1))
 (segment (start 152 102.04) (end 124.54 102.04) (width 0.2) (layer "F.Cu") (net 1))
 (segment (start 124.27 101.77) (end 124.27 99.647794) (width 0.2) (layer "F.Cu") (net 1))
 (segment (start 102.74705 88.5) (end 97.14605 94.101) (width 0.2) (layer "F.Cu") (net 1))
 (segment (start 124.54 102.04) (end 124.27 101.77) (width 0.2) (layer "F.Cu") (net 1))
 (segment (start 95.101 94.101) (end 76 75) (width 0.2) (layer "F.Cu") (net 1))
 (segment (start 154.5 99.54) (end 152 102.04) (width 0.2) (layer "F.Cu") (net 1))
 (segment (start 97.14605 94.101) (end 95.101 94.101) (width 0.2) (layer "F.Cu") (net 1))
 (segment (start 124.27 99.647794) (end 113.122206 88.5) (width 0.2) (layer "F.Cu") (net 1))
 (segment (start 155.701 73.299) (end 153.161 73.299) (width 0.2) (layer "F.Cu") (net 5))
 (segment (start 152.06676 103.601) (end 155.701 99.96676) (width 0.2) (layer "F.Cu") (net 5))
 (segment (start 97.481 103.601) (end 152.06676 103.601) (width 0.2) (layer "F.Cu") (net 5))
 (segment (start 153.161 73.299) (end 151.96 74.5) (width 0.2) (layer "F.Cu") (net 5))
 (segment (start 96.38 102.5) (end 97.481 103.601) (width 0.2) (layer "F.Cu") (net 5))
 (segment (start 155.701 99.96676) (end 155.701 73.299) (width 0.2) (layer "F.Cu") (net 5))
 (segment (start 73.46 75) (end 95.96 97.5) (width 0.2) (layer "F.Cu") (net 2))
 (segment (start 95.96 97.5) (end 96.38 97.5) (width 0.2) (layer "F.Cu") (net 2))
 (segment (start 115.5 93) (end 123 100.5) (width 0.2) (layer "F.Cu") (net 6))
 (segment (start 104.31 93) (end 115.5 93) (width 0.2) (layer "F.Cu") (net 6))
 (segment (start 96.69 78.31) (end 110.5 64.5) (width 0.2) (layer "F.Cu") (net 4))
 (segment (start 96.69 93) (end 96.69 78.31) (width 0.2) (layer "F.Cu") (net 4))
 (segment (start 117 64.5) (end 110.5 64.5) (width 0.2) (layer "F.Cu") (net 4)))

